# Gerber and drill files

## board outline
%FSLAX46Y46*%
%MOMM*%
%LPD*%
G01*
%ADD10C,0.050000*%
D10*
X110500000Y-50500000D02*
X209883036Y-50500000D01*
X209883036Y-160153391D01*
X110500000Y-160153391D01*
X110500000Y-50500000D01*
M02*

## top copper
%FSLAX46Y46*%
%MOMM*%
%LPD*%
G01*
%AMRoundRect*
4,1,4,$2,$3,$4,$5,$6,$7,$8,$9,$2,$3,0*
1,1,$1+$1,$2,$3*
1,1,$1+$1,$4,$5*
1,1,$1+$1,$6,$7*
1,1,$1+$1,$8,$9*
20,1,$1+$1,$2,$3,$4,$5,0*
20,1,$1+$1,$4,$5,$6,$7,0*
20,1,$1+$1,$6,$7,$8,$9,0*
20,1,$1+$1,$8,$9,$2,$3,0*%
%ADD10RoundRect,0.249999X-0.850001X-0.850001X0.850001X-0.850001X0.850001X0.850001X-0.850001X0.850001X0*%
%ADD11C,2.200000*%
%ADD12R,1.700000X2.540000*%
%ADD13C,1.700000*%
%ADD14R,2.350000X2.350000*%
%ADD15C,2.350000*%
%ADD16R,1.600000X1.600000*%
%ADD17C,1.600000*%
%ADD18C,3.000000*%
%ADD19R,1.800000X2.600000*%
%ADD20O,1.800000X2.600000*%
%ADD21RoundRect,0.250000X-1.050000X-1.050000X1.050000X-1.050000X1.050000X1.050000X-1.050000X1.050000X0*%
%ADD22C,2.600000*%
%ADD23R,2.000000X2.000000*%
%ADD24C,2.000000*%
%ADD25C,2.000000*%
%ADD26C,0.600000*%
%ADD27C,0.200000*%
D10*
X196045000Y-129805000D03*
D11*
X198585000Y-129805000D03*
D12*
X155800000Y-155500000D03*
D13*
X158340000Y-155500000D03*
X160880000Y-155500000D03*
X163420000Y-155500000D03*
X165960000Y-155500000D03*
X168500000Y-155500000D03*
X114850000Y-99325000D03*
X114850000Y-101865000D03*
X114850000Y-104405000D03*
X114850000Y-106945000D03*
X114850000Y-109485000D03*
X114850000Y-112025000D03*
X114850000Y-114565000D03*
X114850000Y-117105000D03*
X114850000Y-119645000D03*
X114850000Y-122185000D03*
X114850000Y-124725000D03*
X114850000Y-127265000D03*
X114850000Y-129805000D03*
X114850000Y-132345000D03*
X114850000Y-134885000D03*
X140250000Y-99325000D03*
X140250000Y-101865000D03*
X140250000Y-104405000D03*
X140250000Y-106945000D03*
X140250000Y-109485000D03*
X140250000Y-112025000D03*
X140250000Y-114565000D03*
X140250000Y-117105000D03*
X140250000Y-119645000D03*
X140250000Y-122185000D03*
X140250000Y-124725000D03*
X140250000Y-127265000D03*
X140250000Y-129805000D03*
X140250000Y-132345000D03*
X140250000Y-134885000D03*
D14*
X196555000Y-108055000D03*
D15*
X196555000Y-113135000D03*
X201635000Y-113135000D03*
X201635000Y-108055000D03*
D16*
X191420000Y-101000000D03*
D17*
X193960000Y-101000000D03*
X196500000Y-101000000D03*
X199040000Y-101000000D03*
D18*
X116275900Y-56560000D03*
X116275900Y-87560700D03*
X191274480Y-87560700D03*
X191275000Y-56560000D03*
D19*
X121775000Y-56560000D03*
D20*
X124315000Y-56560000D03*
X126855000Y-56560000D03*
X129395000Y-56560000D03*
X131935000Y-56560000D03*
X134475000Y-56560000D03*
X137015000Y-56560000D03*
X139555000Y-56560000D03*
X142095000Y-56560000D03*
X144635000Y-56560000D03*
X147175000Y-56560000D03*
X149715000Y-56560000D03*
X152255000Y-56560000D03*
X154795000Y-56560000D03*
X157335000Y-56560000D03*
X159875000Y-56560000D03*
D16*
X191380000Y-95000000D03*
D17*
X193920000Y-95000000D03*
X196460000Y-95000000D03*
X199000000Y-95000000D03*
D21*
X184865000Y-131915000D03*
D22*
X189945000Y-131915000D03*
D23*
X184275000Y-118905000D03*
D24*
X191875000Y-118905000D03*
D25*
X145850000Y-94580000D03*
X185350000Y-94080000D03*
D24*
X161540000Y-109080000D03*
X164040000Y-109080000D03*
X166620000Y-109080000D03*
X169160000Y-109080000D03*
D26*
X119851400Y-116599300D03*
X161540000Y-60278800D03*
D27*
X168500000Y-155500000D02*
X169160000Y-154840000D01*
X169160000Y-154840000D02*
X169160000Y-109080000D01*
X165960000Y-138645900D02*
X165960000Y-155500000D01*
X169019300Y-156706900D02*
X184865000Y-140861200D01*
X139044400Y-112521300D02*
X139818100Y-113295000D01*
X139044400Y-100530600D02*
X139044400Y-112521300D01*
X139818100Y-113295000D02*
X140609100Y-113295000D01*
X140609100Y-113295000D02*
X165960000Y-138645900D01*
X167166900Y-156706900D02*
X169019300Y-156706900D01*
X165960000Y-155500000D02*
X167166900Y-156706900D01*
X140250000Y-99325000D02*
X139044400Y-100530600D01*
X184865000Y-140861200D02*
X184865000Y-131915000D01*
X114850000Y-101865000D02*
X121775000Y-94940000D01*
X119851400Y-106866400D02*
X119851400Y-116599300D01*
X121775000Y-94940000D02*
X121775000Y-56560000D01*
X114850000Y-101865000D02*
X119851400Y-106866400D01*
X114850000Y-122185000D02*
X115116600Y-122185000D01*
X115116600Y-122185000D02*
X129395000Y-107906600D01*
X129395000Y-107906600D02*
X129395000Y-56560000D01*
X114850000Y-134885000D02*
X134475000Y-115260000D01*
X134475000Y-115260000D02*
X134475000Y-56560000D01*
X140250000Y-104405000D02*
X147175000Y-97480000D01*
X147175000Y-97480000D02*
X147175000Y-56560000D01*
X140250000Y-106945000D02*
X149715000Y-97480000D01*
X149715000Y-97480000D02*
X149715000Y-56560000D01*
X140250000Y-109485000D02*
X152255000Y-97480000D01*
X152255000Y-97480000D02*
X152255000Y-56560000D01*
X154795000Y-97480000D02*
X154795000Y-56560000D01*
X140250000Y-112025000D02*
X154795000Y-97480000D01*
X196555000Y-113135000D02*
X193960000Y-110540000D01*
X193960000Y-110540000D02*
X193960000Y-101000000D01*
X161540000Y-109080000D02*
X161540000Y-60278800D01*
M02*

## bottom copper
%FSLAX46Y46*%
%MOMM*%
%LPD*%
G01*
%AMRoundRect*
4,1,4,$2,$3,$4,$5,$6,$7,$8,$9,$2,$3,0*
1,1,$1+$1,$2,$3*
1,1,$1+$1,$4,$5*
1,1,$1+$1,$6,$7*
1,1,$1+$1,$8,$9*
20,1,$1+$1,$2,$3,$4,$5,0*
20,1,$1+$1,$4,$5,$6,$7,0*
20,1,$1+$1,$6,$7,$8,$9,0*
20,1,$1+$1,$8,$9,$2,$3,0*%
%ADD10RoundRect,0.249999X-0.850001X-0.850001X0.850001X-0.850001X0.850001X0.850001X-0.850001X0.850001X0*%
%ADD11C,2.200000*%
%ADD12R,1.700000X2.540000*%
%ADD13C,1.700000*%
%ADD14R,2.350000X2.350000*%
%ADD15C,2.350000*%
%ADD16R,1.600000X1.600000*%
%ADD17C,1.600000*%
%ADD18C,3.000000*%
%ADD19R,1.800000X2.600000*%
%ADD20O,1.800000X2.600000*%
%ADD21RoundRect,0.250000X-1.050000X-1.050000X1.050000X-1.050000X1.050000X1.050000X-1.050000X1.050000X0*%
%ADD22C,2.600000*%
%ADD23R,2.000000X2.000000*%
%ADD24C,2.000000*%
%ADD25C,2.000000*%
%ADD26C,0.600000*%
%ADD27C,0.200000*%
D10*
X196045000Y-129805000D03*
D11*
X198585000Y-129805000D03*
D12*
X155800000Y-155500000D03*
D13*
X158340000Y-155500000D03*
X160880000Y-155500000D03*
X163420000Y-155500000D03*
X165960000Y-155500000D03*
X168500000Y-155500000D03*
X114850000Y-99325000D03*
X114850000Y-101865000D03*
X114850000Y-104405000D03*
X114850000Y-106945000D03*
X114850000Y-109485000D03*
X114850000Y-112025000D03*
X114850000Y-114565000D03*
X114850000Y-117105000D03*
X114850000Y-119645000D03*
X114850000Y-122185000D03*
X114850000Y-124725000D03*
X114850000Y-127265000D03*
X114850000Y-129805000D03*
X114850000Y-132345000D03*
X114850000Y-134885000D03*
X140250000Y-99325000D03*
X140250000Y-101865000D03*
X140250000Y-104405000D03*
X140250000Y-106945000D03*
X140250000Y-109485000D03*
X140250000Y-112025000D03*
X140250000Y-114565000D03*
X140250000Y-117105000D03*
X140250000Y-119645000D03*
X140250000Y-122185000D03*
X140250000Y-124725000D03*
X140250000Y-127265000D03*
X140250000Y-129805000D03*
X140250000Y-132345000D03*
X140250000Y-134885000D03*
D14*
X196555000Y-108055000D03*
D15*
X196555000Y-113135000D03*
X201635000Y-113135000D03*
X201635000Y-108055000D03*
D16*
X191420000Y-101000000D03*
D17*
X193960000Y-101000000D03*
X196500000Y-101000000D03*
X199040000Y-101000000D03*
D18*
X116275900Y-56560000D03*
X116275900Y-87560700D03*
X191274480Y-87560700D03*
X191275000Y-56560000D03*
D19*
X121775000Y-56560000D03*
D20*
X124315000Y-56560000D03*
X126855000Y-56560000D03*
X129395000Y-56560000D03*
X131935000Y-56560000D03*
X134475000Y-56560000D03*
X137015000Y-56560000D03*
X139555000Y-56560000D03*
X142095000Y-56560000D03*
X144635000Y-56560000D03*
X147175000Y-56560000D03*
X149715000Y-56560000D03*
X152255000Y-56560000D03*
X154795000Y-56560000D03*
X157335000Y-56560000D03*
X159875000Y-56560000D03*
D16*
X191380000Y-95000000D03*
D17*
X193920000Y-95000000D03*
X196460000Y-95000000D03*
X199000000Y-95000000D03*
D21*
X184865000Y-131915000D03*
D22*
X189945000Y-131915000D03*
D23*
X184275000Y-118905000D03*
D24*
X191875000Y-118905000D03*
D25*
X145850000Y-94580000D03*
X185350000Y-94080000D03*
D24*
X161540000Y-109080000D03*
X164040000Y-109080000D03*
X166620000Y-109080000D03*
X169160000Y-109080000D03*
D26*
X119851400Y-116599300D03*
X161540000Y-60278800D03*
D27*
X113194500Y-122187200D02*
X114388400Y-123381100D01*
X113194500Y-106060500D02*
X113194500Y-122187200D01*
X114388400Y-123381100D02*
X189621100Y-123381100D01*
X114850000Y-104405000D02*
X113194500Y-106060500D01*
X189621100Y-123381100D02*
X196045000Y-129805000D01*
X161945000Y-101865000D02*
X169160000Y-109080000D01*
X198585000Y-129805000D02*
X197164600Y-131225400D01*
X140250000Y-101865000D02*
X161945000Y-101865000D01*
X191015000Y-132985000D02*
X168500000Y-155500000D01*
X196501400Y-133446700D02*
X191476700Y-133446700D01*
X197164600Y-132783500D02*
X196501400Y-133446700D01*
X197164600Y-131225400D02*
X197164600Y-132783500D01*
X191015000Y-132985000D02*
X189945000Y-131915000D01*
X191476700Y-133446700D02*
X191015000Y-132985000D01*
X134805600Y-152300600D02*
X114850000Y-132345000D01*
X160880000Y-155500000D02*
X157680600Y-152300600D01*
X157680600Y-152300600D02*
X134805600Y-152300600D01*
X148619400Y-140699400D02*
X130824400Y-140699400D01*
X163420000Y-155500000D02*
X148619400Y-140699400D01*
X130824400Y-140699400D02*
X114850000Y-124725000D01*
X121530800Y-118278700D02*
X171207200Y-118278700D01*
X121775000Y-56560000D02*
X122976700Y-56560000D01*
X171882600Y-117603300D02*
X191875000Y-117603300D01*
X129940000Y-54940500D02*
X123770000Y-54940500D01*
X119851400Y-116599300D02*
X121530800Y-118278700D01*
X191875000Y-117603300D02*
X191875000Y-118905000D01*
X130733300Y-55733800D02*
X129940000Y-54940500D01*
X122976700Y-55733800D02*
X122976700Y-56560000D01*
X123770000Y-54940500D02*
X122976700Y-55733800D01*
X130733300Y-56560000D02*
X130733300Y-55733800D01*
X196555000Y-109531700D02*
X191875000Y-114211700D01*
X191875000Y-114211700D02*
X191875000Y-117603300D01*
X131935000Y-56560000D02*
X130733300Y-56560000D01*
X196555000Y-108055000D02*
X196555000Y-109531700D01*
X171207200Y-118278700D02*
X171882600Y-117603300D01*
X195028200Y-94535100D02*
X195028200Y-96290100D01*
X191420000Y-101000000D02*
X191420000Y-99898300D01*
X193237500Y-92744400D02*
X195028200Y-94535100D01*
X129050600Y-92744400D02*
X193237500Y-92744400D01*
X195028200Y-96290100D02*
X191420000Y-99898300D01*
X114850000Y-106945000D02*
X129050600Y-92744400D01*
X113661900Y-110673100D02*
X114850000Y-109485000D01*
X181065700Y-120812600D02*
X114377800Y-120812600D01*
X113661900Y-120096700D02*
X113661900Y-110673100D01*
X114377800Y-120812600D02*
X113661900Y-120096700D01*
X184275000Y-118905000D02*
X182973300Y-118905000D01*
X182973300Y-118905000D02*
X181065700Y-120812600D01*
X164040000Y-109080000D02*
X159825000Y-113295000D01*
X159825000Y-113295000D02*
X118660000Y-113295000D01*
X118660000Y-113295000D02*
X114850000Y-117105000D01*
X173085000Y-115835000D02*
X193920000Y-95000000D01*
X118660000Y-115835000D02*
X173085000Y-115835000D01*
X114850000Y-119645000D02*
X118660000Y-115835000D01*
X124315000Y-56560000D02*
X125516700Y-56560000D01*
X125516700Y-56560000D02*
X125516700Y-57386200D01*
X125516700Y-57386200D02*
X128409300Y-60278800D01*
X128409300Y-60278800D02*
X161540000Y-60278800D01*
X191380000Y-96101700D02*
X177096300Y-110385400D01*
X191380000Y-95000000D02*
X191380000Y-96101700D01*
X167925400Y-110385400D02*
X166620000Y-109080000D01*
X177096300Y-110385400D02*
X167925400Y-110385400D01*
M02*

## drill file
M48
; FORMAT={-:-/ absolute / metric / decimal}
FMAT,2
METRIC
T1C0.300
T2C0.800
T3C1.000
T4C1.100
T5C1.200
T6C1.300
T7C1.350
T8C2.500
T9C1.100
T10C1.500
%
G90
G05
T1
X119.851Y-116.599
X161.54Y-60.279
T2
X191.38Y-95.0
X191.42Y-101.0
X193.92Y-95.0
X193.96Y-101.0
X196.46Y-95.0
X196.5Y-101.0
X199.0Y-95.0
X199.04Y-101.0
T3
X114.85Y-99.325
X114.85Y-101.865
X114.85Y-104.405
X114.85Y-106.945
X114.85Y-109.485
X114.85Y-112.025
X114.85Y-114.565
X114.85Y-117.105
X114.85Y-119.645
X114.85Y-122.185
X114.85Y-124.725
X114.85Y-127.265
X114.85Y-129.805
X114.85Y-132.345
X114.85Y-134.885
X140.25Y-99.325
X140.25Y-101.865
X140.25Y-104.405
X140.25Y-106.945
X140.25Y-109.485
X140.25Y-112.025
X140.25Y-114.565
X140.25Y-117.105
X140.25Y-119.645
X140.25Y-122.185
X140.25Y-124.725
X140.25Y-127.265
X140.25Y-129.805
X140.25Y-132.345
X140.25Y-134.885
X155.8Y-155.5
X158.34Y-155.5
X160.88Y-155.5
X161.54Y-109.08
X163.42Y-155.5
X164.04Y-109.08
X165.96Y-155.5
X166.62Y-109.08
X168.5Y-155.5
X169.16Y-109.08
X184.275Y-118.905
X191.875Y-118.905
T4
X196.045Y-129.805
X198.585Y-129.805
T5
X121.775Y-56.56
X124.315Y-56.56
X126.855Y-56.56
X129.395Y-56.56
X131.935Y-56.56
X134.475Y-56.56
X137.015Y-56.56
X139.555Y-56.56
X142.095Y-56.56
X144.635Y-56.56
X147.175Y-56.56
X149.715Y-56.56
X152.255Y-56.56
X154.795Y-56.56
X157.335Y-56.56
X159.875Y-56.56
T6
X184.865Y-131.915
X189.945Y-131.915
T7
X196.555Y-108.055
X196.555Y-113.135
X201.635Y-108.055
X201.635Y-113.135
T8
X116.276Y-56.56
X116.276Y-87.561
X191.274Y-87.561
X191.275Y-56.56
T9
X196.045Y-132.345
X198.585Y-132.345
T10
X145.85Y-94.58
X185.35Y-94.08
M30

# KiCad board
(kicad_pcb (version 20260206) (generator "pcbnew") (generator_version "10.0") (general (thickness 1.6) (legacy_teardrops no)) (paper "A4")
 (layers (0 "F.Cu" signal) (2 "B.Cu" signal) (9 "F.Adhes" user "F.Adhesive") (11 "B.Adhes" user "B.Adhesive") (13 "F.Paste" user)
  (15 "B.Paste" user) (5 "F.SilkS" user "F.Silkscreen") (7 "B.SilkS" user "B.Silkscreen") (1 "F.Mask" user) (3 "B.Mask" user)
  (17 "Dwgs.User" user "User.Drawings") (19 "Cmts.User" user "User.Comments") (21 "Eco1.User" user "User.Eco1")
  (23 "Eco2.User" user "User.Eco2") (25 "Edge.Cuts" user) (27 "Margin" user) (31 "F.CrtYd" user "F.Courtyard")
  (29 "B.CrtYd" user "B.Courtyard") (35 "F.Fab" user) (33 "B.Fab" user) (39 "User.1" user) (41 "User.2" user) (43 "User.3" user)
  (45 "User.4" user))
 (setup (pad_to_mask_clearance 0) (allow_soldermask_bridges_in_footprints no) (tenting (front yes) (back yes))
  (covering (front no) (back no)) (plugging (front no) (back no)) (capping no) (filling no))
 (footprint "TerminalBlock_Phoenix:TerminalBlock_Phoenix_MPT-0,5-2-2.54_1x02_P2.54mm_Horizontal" (layer "F.Cu") (at 196.045 129.805)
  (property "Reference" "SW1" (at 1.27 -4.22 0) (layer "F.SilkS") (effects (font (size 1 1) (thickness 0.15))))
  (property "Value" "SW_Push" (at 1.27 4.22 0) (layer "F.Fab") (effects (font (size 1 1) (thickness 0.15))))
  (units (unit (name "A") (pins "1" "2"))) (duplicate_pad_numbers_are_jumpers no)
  (pad "" np_thru_hole circle (at 0 2.54) (size 1.1 1.1) (drill 1.1) (layers "*.Cu" "*.Mask"))
  (pad "" np_thru_hole circle (at 2.54 2.54) (size 1.1 1.1) (drill 1.1) (layers "*.Cu" "*.Mask"))
  (pad "1" thru_hole roundrect (at 0 0) (size 2.2 2.2) (drill 1.1) (layers "*.Cu" "*.Mask") (remove_unused_layers no)
   (roundrect_rratio 0.113636) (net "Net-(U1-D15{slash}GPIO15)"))
  (pad "2" thru_hole circle (at 2.54 0) (size 2.2 2.2) (drill 1.1) (layers "*.Cu" "*.Mask") (remove_unused_layers no) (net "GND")))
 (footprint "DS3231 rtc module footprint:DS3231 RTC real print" (layer "F.Cu") (at 155.8 155.5 90)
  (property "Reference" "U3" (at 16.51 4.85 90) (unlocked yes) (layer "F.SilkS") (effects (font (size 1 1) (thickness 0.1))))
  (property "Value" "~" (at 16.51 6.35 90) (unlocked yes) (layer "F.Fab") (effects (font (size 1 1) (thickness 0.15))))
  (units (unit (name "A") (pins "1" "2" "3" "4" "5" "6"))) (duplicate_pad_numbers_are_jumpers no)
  (pad "1" thru_hole rect (at 0 0 90) (size 2.54 1.7) (drill 1) (layers "*.Cu" "*.Mask") (remove_unused_layers no)
   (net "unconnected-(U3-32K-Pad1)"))
  (pad "2" thru_hole circle (at 0 2.54 90) (size 1.7 1.7) (drill 1) (layers "*.Cu" "*.Mask") (remove_unused_layers no)
   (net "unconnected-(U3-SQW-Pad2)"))
  (pad "3" thru_hole circle (at 0 5.08 90) (size 1.7 1.7) (drill 1) (layers "*.Cu" "*.Mask") (remove_unused_layers no)
   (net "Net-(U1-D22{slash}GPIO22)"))
  (pad "4" thru_hole circle (at 0 7.62 270) (size 1.7 1.7) (drill 1) (layers "*.Cu" "*.Mask") (remove_unused_layers no)
   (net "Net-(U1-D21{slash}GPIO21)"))
  (pad "5" thru_hole circle (at 0 10.16 90) (size 1.7 1.7) (drill 1) (layers "*.Cu" "*.Mask") (remove_unused_layers no)
   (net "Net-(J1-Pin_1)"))
  (pad "6" thru_hole circle (at 0 12.7 90) (size 1.7 1.7) (drill 1) (layers "*.Cu" "*.Mask") (remove_unused_layers no) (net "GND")))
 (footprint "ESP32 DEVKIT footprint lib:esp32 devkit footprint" (layer "F.Cu") (at 127.55 117.105)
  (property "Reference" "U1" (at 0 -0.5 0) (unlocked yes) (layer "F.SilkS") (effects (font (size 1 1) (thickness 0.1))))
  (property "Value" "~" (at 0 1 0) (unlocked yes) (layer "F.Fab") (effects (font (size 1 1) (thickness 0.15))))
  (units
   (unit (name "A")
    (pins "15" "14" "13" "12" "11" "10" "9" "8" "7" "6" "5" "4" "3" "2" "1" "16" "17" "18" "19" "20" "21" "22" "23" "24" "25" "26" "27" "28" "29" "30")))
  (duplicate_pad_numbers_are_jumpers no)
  (pad "1" thru_hole circle (at -12.7 -17.78 180) (size 1.7 1.7) (drill 1) (layers "*.Cu" "*.Mask") (remove_unused_layers no)
   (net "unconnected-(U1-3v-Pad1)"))
  (pad "2" thru_hole circle (at -12.7 -15.24 180) (size 1.7 1.7) (drill 1) (layers "*.Cu" "*.Mask") (remove_unused_layers no)
   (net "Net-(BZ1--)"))
  (pad "3" thru_hole circle (at -12.7 -12.7 180) (size 1.7 1.7) (drill 1) (layers "*.Cu" "*.Mask") (remove_unused_layers no)
   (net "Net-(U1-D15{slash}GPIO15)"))
  (pad "4" thru_hole circle (at -12.7 -10.16 180) (size 1.7 1.7) (drill 1) (layers "*.Cu" "*.Mask") (remove_unused_layers no)
   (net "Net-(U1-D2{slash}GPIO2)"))
  (pad "5" thru_hole circle (at -12.7 -7.62 180) (size 1.7 1.7) (drill 1) (layers "*.Cu" "*.Mask") (remove_unused_layers no)
   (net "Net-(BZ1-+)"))
  (pad "6" thru_hole circle (at -12.7 -5.08 180) (size 1.7 1.7) (drill 1) (layers "*.Cu" "*.Mask") (remove_unused_layers no)
   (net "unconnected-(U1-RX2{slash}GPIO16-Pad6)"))
  (pad "7" thru_hole circle (at -12.7 -2.54 180) (size 1.7 1.7) (drill 1) (layers "*.Cu" "*.Mask") (remove_unused_layers no)
   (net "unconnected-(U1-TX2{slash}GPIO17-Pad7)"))
  (pad "8" thru_hole circle (at -12.7 0 180) (size 1.7 1.7) (drill 1) (layers "*.Cu" "*.Mask") (remove_unused_layers no)
   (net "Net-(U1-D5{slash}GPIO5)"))
  (pad "9" thru_hole circle (at -12.7 2.54 180) (size 1.7 1.7) (drill 1) (layers "*.Cu" "*.Mask") (remove_unused_layers no)
   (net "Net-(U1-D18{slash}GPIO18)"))
  (pad "10" thru_hole circle (at -12.7 5.08 180) (size 1.7 1.7) (drill 1) (layers "*.Cu" "*.Mask") (remove_unused_layers no)
   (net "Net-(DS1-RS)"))
  (pad "11" thru_hole circle (at -12.7 7.62 180) (size 1.7 1.7) (drill 1) (layers "*.Cu" "*.Mask") (remove_unused_layers no)
   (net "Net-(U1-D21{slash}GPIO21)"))
  (pad "12" thru_hole circle (at -12.7 10.16 180) (size 1.7 1.7) (drill 1) (layers "*.Cu" "*.Mask") (remove_unused_layers no)
   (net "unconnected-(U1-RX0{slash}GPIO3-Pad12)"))
  (pad "13" thru_hole circle (at -12.7 12.7 180) (size 1.7 1.7) (drill 1) (layers "*.Cu" "*.Mask") (remove_unused_layers no)
   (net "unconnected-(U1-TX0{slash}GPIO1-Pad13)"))
  (pad "14" thru_hole circle (at -12.7 15.24 180) (size 1.7 1.7) (drill 1) (layers "*.Cu" "*.Mask") (remove_unused_layers no)
   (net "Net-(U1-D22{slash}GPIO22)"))
  (pad "15" thru_hole circle (at -12.7 17.78 180) (size 1.7 1.7) (drill 1) (layers "*.Cu" "*.Mask") (remove_unused_layers no)
   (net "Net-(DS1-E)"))
  (pad "16" thru_hole circle (at 12.7 -17.78) (size 1.7 1.7) (drill 1) (layers "*.Cu" "*.Mask") (remove_unused_layers no)
   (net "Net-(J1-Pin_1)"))
  (pad "17" thru_hole circle (at 12.7 -15.24) (size 1.7 1.7) (drill 1) (layers "*.Cu" "*.Mask") (remove_unused_layers no) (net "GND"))
  (pad "18" thru_hole circle (at 12.7 -12.7) (size 1.7 1.7) (drill 1) (layers "*.Cu" "*.Mask") (remove_unused_layers no)
   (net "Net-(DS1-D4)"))
  (pad "19" thru_hole circle (at 12.7 -10.16) (size 1.7 1.7) (drill 1) (layers "*.Cu" "*.Mask") (remove_unused_layers no)
   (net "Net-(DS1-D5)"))
  (pad "20" thru_hole circle (at 12.7 -7.62) (size 1.7 1.7) (drill 1) (layers "*.Cu" "*.Mask") (remove_unused_layers no)
   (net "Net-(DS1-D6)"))
  (pad "21" thru_hole circle (at 12.7 -5.08) (size 1.7 1.7) (drill 1) (layers "*.Cu" "*.Mask") (remove_unused_layers no)
   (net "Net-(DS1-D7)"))
  (pad "22" thru_hole circle (at 12.7 -2.54) (size 1.7 1.7) (drill 1) (layers "*.Cu" "*.Mask") (remove_unused_layers no)
   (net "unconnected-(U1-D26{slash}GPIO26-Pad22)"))
  (pad "23" thru_hole circle (at 12.7 0) (size 1.7 1.7) (drill 1) (layers "*.Cu" "*.Mask") (remove_unused_layers no)
   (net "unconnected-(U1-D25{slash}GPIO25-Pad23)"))
  (pad "24" thru_hole circle (at 12.7 2.54) (size 1.7 1.7) (drill 1) (layers "*.Cu" "*.Mask") (remove_unused_layers no)
   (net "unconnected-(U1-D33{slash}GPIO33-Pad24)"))
  (pad "25" thru_hole circle (at 12.7 5.08) (size 1.7 1.7) (drill 1) (layers "*.Cu" "*.Mask") (remove_unused_layers no)
   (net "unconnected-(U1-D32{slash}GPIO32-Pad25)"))
  (pad "26" thru_hole circle (at 12.7 7.62) (size 1.7 1.7) (drill 1) (layers "*.Cu" "*.Mask") (remove_unused_layers no)
   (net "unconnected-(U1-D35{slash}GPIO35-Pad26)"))
  (pad "27" thru_hole circle (at 12.7 10.16) (size 1.7 1.7) (drill 1) (layers "*.Cu" "*.Mask") (remove_unused_layers no)
   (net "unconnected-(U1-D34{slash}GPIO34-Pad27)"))
  (pad "28" thru_hole circle (at 12.7 12.7) (size 1.7 1.7) (drill 1) (layers "*.Cu" "*.Mask") (remove_unused_layers no)
   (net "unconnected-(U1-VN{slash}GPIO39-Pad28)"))
  (pad "29" thru_hole circle (at 12.7 15.24) (size 1.7 1.7) (drill 1) (layers "*.Cu" "*.Mask") (remove_unused_layers no)
   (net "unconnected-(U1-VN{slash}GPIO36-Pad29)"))
  (pad "30" thru_hole circle (at 12.7 17.78) (size 1.7 1.7) (drill 1) (layers "*.Cu" "*.Mask") (remove_unused_layers no)
   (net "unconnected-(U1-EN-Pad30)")))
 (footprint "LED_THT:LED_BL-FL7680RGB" (layer "F.Cu") (at 196.555 108.055)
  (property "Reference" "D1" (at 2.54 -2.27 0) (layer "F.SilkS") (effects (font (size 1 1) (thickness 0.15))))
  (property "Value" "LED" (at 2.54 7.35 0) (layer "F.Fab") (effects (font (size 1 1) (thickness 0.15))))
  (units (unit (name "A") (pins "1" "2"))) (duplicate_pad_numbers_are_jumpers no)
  (pad "1" thru_hole rect (at 0 0) (size 2.35 2.35) (drill 1.35) (layers "*.Cu" "*.Mask") (remove_unused_layers no) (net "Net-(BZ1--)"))
  (pad "2" thru_hole circle (at 0 5.08) (size 2.35 2.35) (drill 1.35) (layers "*.Cu" "*.Mask") (remove_unused_layers no) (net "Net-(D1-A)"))
  (pad "3" thru_hole circle (at 5.08 5.08) (size 2.35 2.35) (drill 1.35) (layers "*.Cu" "*.Mask") (remove_unused_layers no))
  (pad "4" thru_hole circle (at 5.08 0) (size 2.35 2.35) (drill 1.35) (layers "*.Cu" "*.Mask") (remove_unused_layers no)))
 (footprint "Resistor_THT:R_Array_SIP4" (layer "F.Cu") (at 191.42 101)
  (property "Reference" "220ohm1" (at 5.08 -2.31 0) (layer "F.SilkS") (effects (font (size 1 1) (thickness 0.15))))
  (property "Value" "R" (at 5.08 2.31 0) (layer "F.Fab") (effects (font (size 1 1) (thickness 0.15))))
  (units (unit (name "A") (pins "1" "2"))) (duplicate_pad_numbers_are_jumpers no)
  (pad "1" thru_hole rect (at 0 0) (size 1.6 1.6) (drill 0.8) (layers "*.Cu" "*.Mask") (remove_unused_layers no)
   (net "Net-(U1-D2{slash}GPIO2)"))
  (pad "2" thru_hole circle (at 2.54 0) (size 1.6 1.6) (drill 0.8) (layers "*.Cu" "*.Mask") (remove_unused_layers no) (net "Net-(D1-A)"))
  (pad "3" thru_hole circle (at 5.08 0) (size 1.6 1.6) (drill 0.8) (layers "*.Cu" "*.Mask") (remove_unused_layers no))
  (pad "4" thru_hole circle (at 7.62 0) (size 1.6 1.6) (drill 0.8) (layers "*.Cu" "*.Mask") (remove_unused_layers no)))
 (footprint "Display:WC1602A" (layer "F.Cu") (at 121.775 56.56)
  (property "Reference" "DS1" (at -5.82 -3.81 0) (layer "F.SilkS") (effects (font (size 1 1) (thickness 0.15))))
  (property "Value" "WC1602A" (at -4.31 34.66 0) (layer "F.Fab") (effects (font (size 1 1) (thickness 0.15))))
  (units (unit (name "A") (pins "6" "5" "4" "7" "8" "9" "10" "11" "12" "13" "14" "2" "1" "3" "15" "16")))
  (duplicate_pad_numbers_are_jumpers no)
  (pad "" thru_hole circle (at -5.4991 0) (size 3 3) (drill 2.5) (layers "*.Cu" "*.Mask") (remove_unused_layers no))
  (pad "" thru_hole circle (at -5.4991 31.0007) (size 3 3) (drill 2.5) (layers "*.Cu" "*.Mask") (remove_unused_layers no))
  (pad "" thru_hole circle (at 69.49948 31.0007) (size 3 3) (drill 2.5) (layers "*.Cu" "*.Mask") (remove_unused_layers no))
  (pad "" thru_hole circle (at 69.5 0) (size 3 3) (drill 2.5) (layers "*.Cu" "*.Mask") (remove_unused_layers no))
  (pad "1" thru_hole rect (at 0 0) (size 1.8 2.6) (drill 1.2) (layers "*.Cu" "*.Mask") (remove_unused_layers no) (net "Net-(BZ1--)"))
  (pad "2" thru_hole oval (at 2.54 0) (size 1.8 2.6) (drill 1.2) (layers "*.Cu" "*.Mask") (remove_unused_layers no) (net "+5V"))
  (pad "3" thru_hole oval (at 5.08 0) (size 1.8 2.6) (drill 1.2) (layers "*.Cu" "*.Mask") (remove_unused_layers no)
   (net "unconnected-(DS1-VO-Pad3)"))
  (pad "4" thru_hole oval (at 7.62 0) (size 1.8 2.6) (drill 1.2) (layers "*.Cu" "*.Mask") (remove_unused_layers no) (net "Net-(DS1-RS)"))
  (pad "5" thru_hole oval (at 10.16 0) (size 1.8 2.6) (drill 1.2) (layers "*.Cu" "*.Mask") (remove_unused_layers no) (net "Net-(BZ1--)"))
  (pad "6" thru_hole oval (at 12.7 0) (size 1.8 2.6) (drill 1.2) (layers "*.Cu" "*.Mask") (remove_unused_layers no) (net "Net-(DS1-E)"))
  (pad "7" thru_hole oval (at 15.24 0) (size 1.8 2.6) (drill 1.2) (layers "*.Cu" "*.Mask") (remove_unused_layers no)
   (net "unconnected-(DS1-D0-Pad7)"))
  (pad "8" thru_hole oval (at 17.78 0) (size 1.8 2.6) (drill 1.2) (layers "*.Cu" "*.Mask") (remove_unused_layers no)
   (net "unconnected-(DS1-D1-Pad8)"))
  (pad "9" thru_hole oval (at 20.32 0) (size 1.8 2.6) (drill 1.2) (layers "*.Cu" "*.Mask") (remove_unused_layers no)
   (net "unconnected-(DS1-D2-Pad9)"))
  (pad "10" thru_hole oval (at 22.86 0) (size 1.8 2.6) (drill 1.2) (layers "*.Cu" "*.Mask") (remove_unused_layers no)
   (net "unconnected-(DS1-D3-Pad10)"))
  (pad "11" thru_hole oval (at 25.4 0) (size 1.8 2.6) (drill 1.2) (layers "*.Cu" "*.Mask") (remove_unused_layers no) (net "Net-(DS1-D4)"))
  (pad "12" thru_hole oval (at 27.94 0) (size 1.8 2.6) (drill 1.2) (layers "*.Cu" "*.Mask") (remove_unused_layers no) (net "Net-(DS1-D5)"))
  (pad "13" thru_hole oval (at 30.48 0) (size 1.8 2.6) (drill 1.2) (layers "*.Cu" "*.Mask") (remove_unused_layers no) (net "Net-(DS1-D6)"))
  (pad "14" thru_hole oval (at 33.02 0) (size 1.8 2.6) (drill 1.2) (layers "*.Cu" "*.Mask") (remove_unused_layers no) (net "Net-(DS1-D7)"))
  (pad "15" thru_hole oval (at 35.56 0) (size 1.8 2.6) (drill 1.2) (layers "*.Cu" "*.Mask") (remove_unused_layers no)
   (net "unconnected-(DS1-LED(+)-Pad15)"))
  (pad "16" thru_hole oval (at 38.1 0) (size 1.8 2.6) (drill 1.2) (layers "*.Cu" "*.Mask") (remove_unused_layers no)
   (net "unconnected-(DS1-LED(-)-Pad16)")))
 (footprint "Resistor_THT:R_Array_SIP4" (layer "F.Cu") (at 191.38 95)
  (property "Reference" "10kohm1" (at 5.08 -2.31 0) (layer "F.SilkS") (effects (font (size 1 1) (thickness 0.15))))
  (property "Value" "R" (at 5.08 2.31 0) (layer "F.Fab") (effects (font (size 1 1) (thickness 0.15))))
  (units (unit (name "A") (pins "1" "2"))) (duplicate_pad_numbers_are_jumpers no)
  (pad "1" thru_hole rect (at 0 0) (size 1.6 1.6) (drill 0.8) (layers "*.Cu" "*.Mask") (remove_unused_layers no) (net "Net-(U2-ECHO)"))
  (pad "2" thru_hole circle (at 2.54 0) (size 1.6 1.6) (drill 0.8) (layers "*.Cu" "*.Mask") (remove_unused_layers no)
   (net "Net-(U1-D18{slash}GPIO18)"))
  (pad "3" thru_hole circle (at 5.08 0) (size 1.6 1.6) (drill 0.8) (layers "*.Cu" "*.Mask") (remove_unused_layers no))
  (pad "4" thru_hole circle (at 7.62 0) (size 1.6 1.6) (drill 0.8) (layers "*.Cu" "*.Mask") (remove_unused_layers no)))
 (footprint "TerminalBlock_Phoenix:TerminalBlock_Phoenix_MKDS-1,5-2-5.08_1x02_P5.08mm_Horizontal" (layer "F.Cu") (at 184.865 131.915)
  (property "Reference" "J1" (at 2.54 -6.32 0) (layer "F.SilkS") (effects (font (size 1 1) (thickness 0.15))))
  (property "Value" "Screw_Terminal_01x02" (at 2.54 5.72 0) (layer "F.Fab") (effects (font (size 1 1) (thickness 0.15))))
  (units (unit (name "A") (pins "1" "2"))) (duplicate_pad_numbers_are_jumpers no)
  (pad "1" thru_hole roundrect (at 0 0) (size 2.6 2.6) (drill 1.3) (layers "*.Cu" "*.Mask") (remove_unused_layers no)
   (roundrect_rratio 0.096154) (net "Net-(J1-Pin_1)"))
  (pad "2" thru_hole circle (at 5.08 0) (size 2.6 2.6) (drill 1.3) (layers "*.Cu" "*.Mask") (remove_unused_layers no) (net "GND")))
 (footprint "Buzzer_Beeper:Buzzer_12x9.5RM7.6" (layer "F.Cu") (at 184.275 118.905)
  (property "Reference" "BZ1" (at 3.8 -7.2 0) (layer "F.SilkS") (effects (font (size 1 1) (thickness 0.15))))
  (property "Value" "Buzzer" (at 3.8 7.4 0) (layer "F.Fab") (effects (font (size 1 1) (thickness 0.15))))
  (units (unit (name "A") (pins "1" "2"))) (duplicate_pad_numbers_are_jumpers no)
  (pad "1" thru_hole rect (at 0 0) (size 2 2) (drill 1) (layers "*.Cu" "*.Mask") (remove_unused_layers no) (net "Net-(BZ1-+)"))
  (pad "2" thru_hole circle (at 7.6 0) (size 2 2) (drill 1) (layers "*.Cu" "*.Mask") (remove_unused_layers no) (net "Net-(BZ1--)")))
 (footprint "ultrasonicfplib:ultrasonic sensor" (layer "F.Cu") (at 142.85 91.58)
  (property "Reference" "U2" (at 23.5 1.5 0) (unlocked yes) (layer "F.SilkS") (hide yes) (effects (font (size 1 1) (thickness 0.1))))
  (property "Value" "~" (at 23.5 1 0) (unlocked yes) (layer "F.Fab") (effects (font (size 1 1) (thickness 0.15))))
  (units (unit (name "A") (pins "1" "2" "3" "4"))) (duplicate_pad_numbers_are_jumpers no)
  (pad "" np_thru_hole circle (at 3 3) (size 2 2) (drill 1.5) (layers "*.Cu" "*.Mask"))
  (pad "" np_thru_hole circle (at 42.5 2.5) (size 2 2) (drill 1.5) (layers "*.Cu" "*.Mask"))
  (pad "1" thru_hole circle (at 18.69 17.5) (size 2 2) (drill 1) (layers "*.Cu" "*.Mask") (remove_unused_layers no) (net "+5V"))
  (pad "2" thru_hole circle (at 21.19 17.5) (size 2 2) (drill 1) (layers "*.Cu" "*.Mask") (remove_unused_layers no)
   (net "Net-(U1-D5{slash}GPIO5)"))
  (pad "3" thru_hole circle (at 23.77 17.5) (size 2 2) (drill 1) (layers "*.Cu" "*.Mask") (remove_unused_layers no) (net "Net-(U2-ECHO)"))
  (pad "4" thru_hole circle (at 26.31 17.5) (size 2 2) (drill 1) (layers "*.Cu" "*.Mask") (remove_unused_layers no) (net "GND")))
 (gr_rect (start 110.5 50.5) (end 209.883036 160.153391) (stroke (width 0.05) (type default)) (fill no) (layer "Edge.Cuts"))
 (segment (start 113.1945 122.1872) (end 114.3884 123.3811) (width 0.2) (layer "B.Cu") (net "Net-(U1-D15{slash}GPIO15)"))
 (segment (start 113.1945 106.0605) (end 113.1945 122.1872) (width 0.2) (layer "B.Cu") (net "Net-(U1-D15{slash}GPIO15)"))
 (segment (start 114.3884 123.3811) (end 189.6211 123.3811) (width 0.2) (layer "B.Cu") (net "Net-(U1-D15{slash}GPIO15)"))
 (segment (start 114.85 104.405) (end 113.1945 106.0605) (width 0.2) (layer "B.Cu") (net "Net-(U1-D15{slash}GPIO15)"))
 (segment (start 189.6211 123.3811) (end 196.045 129.805) (width 0.2) (layer "B.Cu") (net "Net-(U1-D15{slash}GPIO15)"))
 (segment (start 168.5 155.5) (end 169.16 154.84) (width 0.2) (layer "F.Cu") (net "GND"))
 (segment (start 169.16 154.84) (end 169.16 109.08) (width 0.2) (layer "F.Cu") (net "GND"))
 (segment (start 161.945 101.865) (end 169.16 109.08) (width 0.2) (layer "B.Cu") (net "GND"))
 (segment (start 198.585 129.805) (end 197.1646 131.2254) (width 0.2) (layer "B.Cu") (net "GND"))
 (segment (start 140.25 101.865) (end 161.945 101.865) (width 0.2) (layer "B.Cu") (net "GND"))
 (segment (start 191.015 132.985) (end 168.5 155.5) (width 0.2) (layer "B.Cu") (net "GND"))
 (segment (start 196.5014 133.4467) (end 191.4767 133.4467) (width 0.2) (layer "B.Cu") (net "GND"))
 (segment (start 197.1646 132.7835) (end 196.5014 133.4467) (width 0.2) (layer "B.Cu") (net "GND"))
 (segment (start 197.1646 131.2254) (end 197.1646 132.7835) (width 0.2) (layer "B.Cu") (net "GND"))
 (segment (start 191.015 132.985) (end 189.945 131.915) (width 0.2) (layer "B.Cu") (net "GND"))
 (segment (start 191.4767 133.4467) (end 191.015 132.985) (width 0.2) (layer "B.Cu") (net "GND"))
 (segment (start 134.8056 152.3006) (end 114.85 132.345) (width 0.2) (layer "B.Cu") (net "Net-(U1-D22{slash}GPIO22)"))
 (segment (start 160.88 155.5) (end 157.6806 152.3006) (width 0.2) (layer "B.Cu") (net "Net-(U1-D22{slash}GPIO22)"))
 (segment (start 157.6806 152.3006) (end 134.8056 152.3006) (width 0.2) (layer "B.Cu") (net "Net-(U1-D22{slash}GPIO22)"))
 (segment (start 148.6194 140.6994) (end 130.8244 140.6994) (width 0.2) (layer "B.Cu") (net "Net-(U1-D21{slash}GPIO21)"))
 (segment (start 163.42 155.5) (end 148.6194 140.6994) (width 0.2) (layer "B.Cu") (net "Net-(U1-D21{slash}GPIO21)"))
 (segment (start 130.8244 140.6994) (end 114.85 124.725) (width 0.2) (layer "B.Cu") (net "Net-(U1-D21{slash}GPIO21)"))
 (segment (start 165.96 138.6459) (end 165.96 155.5) (width 0.2) (layer "F.Cu") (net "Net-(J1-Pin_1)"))
 (segment (start 169.0193 156.7069) (end 184.865 140.8612) (width 0.2) (layer "F.Cu") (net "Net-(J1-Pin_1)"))
 (segment (start 139.0444 112.5213) (end 139.8181 113.295) (width 0.2) (layer "F.Cu") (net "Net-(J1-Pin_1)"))
 (segment (start 139.0444 100.5306) (end 139.0444 112.5213) (width 0.2) (layer "F.Cu") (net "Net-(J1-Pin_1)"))
 (segment (start 139.8181 113.295) (end 140.6091 113.295) (width 0.2) (layer "F.Cu") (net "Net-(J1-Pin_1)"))
 (segment (start 140.6091 113.295) (end 165.96 138.6459) (width 0.2) (layer "F.Cu") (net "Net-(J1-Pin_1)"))
 (segment (start 167.1669 156.7069) (end 169.0193 156.7069) (width 0.2) (layer "F.Cu") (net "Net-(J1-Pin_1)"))
 (segment (start 165.96 155.5) (end 167.1669 156.7069) (width 0.2) (layer "F.Cu") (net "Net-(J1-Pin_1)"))
 (segment (start 140.25 99.325) (end 139.0444 100.5306) (width 0.2) (layer "F.Cu") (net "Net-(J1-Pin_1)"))
 (segment (start 184.865 140.8612) (end 184.865 131.915) (width 0.2) (layer "F.Cu") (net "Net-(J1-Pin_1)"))
 (segment (start 114.85 101.865) (end 121.775 94.94) (width 0.2) (layer "F.Cu") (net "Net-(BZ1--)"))
 (segment (start 119.8514 106.8664) (end 119.8514 116.5993) (width 0.2) (layer "F.Cu") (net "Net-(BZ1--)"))
 (segment (start 121.775 94.94) (end 121.775 56.56) (width 0.2) (layer "F.Cu") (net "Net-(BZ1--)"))
 (segment (start 114.85 101.865) (end 119.8514 106.8664) (width 0.2) (layer "F.Cu") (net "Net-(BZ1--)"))
 (via (at 119.8514 116.5993) (size 0.6) (drill 0.3) (layers "F.Cu" "B.Cu") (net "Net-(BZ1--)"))
 (segment (start 121.5308 118.2787) (end 171.2072 118.2787) (width 0.2) (layer "B.Cu") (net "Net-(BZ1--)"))
 (segment (start 121.775 56.56) (end 122.9767 56.56) (width 0.2) (layer "B.Cu") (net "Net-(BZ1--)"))
 (segment (start 171.8826 117.6033) (end 191.875 117.6033) (width 0.2) (layer "B.Cu") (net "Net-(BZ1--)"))
 (segment (start 129.94 54.9405) (end 123.77 54.9405) (width 0.2) (layer "B.Cu") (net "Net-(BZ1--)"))
 (segment (start 119.8514 116.5993) (end 121.5308 118.2787) (width 0.2) (layer "B.Cu") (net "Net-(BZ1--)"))
 (segment (start 191.875 117.6033) (end 191.875 118.905) (width 0.2) (layer "B.Cu") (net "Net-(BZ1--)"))
 (segment (start 130.7333 55.7338) (end 129.94 54.9405) (width 0.2) (layer "B.Cu") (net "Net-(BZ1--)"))
 (segment (start 122.9767 55.7338) (end 122.9767 56.56) (width 0.2) (layer "B.Cu") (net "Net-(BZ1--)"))
 (segment (start 123.77 54.9405) (end 122.9767 55.7338) (width 0.2) (layer "B.Cu") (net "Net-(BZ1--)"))
 (segment (start 130.7333 56.56) (end 130.7333 55.7338) (width 0.2) (layer "B.Cu") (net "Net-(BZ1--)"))
 (segment (start 196.555 109.5317) (end 191.875 114.2117) (width 0.2) (layer "B.Cu") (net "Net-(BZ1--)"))
 (segment (start 191.875 114.2117) (end 191.875 117.6033) (width 0.2) (layer "B.Cu") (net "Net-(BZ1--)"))
 (segment (start 131.935 56.56) (end 130.7333 56.56) (width 0.2) (layer "B.Cu") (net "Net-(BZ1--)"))
 (segment (start 196.555 108.055) (end 196.555 109.5317) (width 0.2) (layer "B.Cu") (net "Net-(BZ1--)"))
 (segment (start 171.2072 118.2787) (end 171.8826 117.6033) (width 0.2) (layer "B.Cu") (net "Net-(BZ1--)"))
 (segment (start 195.0282 94.5351) (end 195.0282 96.2901) (width 0.2) (layer "B.Cu") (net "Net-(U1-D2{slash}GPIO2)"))
 (segment (start 191.42 101) (end 191.42 99.8983) (width 0.2) (layer "B.Cu") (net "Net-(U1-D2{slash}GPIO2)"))
 (segment (start 193.2375 92.7444) (end 195.0282 94.5351) (width 0.2) (layer "B.Cu") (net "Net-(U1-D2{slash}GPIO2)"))
 (segment (start 129.0506 92.7444) (end 193.2375 92.7444) (width 0.2) (layer "B.Cu") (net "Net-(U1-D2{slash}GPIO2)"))
 (segment (start 195.0282 96.2901) (end 191.42 99.8983) (width 0.2) (layer "B.Cu") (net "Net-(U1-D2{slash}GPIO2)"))
 (segment (start 114.85 106.945) (end 129.0506 92.7444) (width 0.2) (layer "B.Cu") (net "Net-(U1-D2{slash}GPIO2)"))
 (segment (start 113.6619 110.6731) (end 114.85 109.485) (width 0.2) (layer "B.Cu") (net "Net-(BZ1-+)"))
 (segment (start 181.0657 120.8126) (end 114.3778 120.8126) (width 0.2) (layer "B.Cu") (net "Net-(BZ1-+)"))
 (segment (start 113.6619 120.0967) (end 113.6619 110.6731) (width 0.2) (layer "B.Cu") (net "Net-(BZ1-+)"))
 (segment (start 114.3778 120.8126) (end 113.6619 120.0967) (width 0.2) (layer "B.Cu") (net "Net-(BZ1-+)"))
 (segment (start 184.275 118.905) (end 182.9733 118.905) (width 0.2) (layer "B.Cu") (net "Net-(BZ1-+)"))
 (segment (start 182.9733 118.905) (end 181.0657 120.8126) (width 0.2) (layer "B.Cu") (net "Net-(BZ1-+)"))
 (segment (start 164.04 109.08) (end 159.825 113.295) (width 0.2) (layer "B.Cu") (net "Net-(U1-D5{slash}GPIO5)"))
 (segment (start 159.825 113.295) (end 118.66 113.295) (width 0.2) (layer "B.Cu") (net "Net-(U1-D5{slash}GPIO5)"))
 (segment (start 118.66 113.295) (end 114.85 117.105) (width 0.2) (layer "B.Cu") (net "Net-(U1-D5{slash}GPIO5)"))
 (segment (start 173.085 115.835) (end 193.92 95) (width 0.2) (layer "B.Cu") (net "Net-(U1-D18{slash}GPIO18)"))
 (segment (start 118.66 115.835) (end 173.085 115.835) (width 0.2) (layer "B.Cu") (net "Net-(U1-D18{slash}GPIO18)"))
 (segment (start 114.85 119.645) (end 118.66 115.835) (width 0.2) (layer "B.Cu") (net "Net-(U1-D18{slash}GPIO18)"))
 (segment (start 114.85 122.185) (end 115.1166 122.185) (width 0.2) (layer "F.Cu") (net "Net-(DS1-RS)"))
 (segment (start 115.1166 122.185) (end 129.395 107.9066) (width 0.2) (layer "F.Cu") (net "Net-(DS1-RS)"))
 (segment (start 129.395 107.9066) (end 129.395 56.56) (width 0.2) (layer "F.Cu") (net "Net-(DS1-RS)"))
 (segment (start 114.85 134.885) (end 134.475 115.26) (width 0.2) (layer "F.Cu") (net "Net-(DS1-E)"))
 (segment (start 134.475 115.26) (end 134.475 56.56) (width 0.2) (layer "F.Cu") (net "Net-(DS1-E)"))
 (segment (start 140.25 104.405) (end 147.175 97.48) (width 0.2) (layer "F.Cu") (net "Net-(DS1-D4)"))
 (segment (start 147.175 97.48) (end 147.175 56.56) (width 0.2) (layer "F.Cu") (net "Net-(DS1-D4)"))
 (segment (start 140.25 106.945) (end 149.715 97.48) (width 0.2) (layer "F.Cu") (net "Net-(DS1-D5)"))
 (segment (start 149.715 97.48) (end 149.715 56.56) (width 0.2) (layer "F.Cu") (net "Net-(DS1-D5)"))
 (segment (start 140.25 109.485) (end 152.255 97.48) (width 0.2) (layer "F.Cu") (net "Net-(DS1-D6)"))
 (segment (start 152.255 97.48) (end 152.255 56.56) (width 0.2) (layer "F.Cu") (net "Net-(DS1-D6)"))
 (segment (start 154.795 97.48) (end 154.795 56.56) (width 0.2) (layer "F.Cu") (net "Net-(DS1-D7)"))
 (segment (start 140.25 112.025) (end 154.795 97.48) (width 0.2) (layer "F.Cu") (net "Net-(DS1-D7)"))
 (segment (start 196.555 113.135) (end 193.96 110.54) (width 0.2) (layer "F.Cu") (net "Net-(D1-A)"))
 (segment (start 193.96 110.54) (end 193.96 101) (width 0.2) (layer "F.Cu") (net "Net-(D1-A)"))
 (segment (start 161.54 109.08) (end 161.54 60.2788) (width 0.2) (layer "F.Cu") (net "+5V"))
 (via (at 161.54 60.2788) (size 0.6) (drill 0.3) (layers "F.Cu" "B.Cu") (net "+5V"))
 (segment (start 124.315 56.56) (end 125.5167 56.56) (width 0.2) (layer "B.Cu") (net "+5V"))
 (segment (start 125.5167 56.56) (end 125.5167 57.3862) (width 0.2) (layer "B.Cu") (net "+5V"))
 (segment (start 125.5167 57.3862) (end 128.4093 60.2788) (width 0.2) (layer "B.Cu") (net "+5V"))
 (segment (start 128.4093 60.2788) (end 161.54 60.2788) (width 0.2) (layer "B.Cu") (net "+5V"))
 (segment (start 191.38 96.1017) (end 177.0963 110.3854) (width 0.2) (layer "B.Cu") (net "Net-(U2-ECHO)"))
 (segment (start 191.38 95) (end 191.38 96.1017) (width 0.2) (layer "B.Cu") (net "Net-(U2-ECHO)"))
 (segment (start 167.9254 110.3854) (end 166.62 109.08) (width 0.2) (layer "B.Cu") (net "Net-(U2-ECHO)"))
 (segment (start 177.0963 110.3854) (end 167.9254 110.3854) (width 0.2) (layer "B.Cu") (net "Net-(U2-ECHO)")))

